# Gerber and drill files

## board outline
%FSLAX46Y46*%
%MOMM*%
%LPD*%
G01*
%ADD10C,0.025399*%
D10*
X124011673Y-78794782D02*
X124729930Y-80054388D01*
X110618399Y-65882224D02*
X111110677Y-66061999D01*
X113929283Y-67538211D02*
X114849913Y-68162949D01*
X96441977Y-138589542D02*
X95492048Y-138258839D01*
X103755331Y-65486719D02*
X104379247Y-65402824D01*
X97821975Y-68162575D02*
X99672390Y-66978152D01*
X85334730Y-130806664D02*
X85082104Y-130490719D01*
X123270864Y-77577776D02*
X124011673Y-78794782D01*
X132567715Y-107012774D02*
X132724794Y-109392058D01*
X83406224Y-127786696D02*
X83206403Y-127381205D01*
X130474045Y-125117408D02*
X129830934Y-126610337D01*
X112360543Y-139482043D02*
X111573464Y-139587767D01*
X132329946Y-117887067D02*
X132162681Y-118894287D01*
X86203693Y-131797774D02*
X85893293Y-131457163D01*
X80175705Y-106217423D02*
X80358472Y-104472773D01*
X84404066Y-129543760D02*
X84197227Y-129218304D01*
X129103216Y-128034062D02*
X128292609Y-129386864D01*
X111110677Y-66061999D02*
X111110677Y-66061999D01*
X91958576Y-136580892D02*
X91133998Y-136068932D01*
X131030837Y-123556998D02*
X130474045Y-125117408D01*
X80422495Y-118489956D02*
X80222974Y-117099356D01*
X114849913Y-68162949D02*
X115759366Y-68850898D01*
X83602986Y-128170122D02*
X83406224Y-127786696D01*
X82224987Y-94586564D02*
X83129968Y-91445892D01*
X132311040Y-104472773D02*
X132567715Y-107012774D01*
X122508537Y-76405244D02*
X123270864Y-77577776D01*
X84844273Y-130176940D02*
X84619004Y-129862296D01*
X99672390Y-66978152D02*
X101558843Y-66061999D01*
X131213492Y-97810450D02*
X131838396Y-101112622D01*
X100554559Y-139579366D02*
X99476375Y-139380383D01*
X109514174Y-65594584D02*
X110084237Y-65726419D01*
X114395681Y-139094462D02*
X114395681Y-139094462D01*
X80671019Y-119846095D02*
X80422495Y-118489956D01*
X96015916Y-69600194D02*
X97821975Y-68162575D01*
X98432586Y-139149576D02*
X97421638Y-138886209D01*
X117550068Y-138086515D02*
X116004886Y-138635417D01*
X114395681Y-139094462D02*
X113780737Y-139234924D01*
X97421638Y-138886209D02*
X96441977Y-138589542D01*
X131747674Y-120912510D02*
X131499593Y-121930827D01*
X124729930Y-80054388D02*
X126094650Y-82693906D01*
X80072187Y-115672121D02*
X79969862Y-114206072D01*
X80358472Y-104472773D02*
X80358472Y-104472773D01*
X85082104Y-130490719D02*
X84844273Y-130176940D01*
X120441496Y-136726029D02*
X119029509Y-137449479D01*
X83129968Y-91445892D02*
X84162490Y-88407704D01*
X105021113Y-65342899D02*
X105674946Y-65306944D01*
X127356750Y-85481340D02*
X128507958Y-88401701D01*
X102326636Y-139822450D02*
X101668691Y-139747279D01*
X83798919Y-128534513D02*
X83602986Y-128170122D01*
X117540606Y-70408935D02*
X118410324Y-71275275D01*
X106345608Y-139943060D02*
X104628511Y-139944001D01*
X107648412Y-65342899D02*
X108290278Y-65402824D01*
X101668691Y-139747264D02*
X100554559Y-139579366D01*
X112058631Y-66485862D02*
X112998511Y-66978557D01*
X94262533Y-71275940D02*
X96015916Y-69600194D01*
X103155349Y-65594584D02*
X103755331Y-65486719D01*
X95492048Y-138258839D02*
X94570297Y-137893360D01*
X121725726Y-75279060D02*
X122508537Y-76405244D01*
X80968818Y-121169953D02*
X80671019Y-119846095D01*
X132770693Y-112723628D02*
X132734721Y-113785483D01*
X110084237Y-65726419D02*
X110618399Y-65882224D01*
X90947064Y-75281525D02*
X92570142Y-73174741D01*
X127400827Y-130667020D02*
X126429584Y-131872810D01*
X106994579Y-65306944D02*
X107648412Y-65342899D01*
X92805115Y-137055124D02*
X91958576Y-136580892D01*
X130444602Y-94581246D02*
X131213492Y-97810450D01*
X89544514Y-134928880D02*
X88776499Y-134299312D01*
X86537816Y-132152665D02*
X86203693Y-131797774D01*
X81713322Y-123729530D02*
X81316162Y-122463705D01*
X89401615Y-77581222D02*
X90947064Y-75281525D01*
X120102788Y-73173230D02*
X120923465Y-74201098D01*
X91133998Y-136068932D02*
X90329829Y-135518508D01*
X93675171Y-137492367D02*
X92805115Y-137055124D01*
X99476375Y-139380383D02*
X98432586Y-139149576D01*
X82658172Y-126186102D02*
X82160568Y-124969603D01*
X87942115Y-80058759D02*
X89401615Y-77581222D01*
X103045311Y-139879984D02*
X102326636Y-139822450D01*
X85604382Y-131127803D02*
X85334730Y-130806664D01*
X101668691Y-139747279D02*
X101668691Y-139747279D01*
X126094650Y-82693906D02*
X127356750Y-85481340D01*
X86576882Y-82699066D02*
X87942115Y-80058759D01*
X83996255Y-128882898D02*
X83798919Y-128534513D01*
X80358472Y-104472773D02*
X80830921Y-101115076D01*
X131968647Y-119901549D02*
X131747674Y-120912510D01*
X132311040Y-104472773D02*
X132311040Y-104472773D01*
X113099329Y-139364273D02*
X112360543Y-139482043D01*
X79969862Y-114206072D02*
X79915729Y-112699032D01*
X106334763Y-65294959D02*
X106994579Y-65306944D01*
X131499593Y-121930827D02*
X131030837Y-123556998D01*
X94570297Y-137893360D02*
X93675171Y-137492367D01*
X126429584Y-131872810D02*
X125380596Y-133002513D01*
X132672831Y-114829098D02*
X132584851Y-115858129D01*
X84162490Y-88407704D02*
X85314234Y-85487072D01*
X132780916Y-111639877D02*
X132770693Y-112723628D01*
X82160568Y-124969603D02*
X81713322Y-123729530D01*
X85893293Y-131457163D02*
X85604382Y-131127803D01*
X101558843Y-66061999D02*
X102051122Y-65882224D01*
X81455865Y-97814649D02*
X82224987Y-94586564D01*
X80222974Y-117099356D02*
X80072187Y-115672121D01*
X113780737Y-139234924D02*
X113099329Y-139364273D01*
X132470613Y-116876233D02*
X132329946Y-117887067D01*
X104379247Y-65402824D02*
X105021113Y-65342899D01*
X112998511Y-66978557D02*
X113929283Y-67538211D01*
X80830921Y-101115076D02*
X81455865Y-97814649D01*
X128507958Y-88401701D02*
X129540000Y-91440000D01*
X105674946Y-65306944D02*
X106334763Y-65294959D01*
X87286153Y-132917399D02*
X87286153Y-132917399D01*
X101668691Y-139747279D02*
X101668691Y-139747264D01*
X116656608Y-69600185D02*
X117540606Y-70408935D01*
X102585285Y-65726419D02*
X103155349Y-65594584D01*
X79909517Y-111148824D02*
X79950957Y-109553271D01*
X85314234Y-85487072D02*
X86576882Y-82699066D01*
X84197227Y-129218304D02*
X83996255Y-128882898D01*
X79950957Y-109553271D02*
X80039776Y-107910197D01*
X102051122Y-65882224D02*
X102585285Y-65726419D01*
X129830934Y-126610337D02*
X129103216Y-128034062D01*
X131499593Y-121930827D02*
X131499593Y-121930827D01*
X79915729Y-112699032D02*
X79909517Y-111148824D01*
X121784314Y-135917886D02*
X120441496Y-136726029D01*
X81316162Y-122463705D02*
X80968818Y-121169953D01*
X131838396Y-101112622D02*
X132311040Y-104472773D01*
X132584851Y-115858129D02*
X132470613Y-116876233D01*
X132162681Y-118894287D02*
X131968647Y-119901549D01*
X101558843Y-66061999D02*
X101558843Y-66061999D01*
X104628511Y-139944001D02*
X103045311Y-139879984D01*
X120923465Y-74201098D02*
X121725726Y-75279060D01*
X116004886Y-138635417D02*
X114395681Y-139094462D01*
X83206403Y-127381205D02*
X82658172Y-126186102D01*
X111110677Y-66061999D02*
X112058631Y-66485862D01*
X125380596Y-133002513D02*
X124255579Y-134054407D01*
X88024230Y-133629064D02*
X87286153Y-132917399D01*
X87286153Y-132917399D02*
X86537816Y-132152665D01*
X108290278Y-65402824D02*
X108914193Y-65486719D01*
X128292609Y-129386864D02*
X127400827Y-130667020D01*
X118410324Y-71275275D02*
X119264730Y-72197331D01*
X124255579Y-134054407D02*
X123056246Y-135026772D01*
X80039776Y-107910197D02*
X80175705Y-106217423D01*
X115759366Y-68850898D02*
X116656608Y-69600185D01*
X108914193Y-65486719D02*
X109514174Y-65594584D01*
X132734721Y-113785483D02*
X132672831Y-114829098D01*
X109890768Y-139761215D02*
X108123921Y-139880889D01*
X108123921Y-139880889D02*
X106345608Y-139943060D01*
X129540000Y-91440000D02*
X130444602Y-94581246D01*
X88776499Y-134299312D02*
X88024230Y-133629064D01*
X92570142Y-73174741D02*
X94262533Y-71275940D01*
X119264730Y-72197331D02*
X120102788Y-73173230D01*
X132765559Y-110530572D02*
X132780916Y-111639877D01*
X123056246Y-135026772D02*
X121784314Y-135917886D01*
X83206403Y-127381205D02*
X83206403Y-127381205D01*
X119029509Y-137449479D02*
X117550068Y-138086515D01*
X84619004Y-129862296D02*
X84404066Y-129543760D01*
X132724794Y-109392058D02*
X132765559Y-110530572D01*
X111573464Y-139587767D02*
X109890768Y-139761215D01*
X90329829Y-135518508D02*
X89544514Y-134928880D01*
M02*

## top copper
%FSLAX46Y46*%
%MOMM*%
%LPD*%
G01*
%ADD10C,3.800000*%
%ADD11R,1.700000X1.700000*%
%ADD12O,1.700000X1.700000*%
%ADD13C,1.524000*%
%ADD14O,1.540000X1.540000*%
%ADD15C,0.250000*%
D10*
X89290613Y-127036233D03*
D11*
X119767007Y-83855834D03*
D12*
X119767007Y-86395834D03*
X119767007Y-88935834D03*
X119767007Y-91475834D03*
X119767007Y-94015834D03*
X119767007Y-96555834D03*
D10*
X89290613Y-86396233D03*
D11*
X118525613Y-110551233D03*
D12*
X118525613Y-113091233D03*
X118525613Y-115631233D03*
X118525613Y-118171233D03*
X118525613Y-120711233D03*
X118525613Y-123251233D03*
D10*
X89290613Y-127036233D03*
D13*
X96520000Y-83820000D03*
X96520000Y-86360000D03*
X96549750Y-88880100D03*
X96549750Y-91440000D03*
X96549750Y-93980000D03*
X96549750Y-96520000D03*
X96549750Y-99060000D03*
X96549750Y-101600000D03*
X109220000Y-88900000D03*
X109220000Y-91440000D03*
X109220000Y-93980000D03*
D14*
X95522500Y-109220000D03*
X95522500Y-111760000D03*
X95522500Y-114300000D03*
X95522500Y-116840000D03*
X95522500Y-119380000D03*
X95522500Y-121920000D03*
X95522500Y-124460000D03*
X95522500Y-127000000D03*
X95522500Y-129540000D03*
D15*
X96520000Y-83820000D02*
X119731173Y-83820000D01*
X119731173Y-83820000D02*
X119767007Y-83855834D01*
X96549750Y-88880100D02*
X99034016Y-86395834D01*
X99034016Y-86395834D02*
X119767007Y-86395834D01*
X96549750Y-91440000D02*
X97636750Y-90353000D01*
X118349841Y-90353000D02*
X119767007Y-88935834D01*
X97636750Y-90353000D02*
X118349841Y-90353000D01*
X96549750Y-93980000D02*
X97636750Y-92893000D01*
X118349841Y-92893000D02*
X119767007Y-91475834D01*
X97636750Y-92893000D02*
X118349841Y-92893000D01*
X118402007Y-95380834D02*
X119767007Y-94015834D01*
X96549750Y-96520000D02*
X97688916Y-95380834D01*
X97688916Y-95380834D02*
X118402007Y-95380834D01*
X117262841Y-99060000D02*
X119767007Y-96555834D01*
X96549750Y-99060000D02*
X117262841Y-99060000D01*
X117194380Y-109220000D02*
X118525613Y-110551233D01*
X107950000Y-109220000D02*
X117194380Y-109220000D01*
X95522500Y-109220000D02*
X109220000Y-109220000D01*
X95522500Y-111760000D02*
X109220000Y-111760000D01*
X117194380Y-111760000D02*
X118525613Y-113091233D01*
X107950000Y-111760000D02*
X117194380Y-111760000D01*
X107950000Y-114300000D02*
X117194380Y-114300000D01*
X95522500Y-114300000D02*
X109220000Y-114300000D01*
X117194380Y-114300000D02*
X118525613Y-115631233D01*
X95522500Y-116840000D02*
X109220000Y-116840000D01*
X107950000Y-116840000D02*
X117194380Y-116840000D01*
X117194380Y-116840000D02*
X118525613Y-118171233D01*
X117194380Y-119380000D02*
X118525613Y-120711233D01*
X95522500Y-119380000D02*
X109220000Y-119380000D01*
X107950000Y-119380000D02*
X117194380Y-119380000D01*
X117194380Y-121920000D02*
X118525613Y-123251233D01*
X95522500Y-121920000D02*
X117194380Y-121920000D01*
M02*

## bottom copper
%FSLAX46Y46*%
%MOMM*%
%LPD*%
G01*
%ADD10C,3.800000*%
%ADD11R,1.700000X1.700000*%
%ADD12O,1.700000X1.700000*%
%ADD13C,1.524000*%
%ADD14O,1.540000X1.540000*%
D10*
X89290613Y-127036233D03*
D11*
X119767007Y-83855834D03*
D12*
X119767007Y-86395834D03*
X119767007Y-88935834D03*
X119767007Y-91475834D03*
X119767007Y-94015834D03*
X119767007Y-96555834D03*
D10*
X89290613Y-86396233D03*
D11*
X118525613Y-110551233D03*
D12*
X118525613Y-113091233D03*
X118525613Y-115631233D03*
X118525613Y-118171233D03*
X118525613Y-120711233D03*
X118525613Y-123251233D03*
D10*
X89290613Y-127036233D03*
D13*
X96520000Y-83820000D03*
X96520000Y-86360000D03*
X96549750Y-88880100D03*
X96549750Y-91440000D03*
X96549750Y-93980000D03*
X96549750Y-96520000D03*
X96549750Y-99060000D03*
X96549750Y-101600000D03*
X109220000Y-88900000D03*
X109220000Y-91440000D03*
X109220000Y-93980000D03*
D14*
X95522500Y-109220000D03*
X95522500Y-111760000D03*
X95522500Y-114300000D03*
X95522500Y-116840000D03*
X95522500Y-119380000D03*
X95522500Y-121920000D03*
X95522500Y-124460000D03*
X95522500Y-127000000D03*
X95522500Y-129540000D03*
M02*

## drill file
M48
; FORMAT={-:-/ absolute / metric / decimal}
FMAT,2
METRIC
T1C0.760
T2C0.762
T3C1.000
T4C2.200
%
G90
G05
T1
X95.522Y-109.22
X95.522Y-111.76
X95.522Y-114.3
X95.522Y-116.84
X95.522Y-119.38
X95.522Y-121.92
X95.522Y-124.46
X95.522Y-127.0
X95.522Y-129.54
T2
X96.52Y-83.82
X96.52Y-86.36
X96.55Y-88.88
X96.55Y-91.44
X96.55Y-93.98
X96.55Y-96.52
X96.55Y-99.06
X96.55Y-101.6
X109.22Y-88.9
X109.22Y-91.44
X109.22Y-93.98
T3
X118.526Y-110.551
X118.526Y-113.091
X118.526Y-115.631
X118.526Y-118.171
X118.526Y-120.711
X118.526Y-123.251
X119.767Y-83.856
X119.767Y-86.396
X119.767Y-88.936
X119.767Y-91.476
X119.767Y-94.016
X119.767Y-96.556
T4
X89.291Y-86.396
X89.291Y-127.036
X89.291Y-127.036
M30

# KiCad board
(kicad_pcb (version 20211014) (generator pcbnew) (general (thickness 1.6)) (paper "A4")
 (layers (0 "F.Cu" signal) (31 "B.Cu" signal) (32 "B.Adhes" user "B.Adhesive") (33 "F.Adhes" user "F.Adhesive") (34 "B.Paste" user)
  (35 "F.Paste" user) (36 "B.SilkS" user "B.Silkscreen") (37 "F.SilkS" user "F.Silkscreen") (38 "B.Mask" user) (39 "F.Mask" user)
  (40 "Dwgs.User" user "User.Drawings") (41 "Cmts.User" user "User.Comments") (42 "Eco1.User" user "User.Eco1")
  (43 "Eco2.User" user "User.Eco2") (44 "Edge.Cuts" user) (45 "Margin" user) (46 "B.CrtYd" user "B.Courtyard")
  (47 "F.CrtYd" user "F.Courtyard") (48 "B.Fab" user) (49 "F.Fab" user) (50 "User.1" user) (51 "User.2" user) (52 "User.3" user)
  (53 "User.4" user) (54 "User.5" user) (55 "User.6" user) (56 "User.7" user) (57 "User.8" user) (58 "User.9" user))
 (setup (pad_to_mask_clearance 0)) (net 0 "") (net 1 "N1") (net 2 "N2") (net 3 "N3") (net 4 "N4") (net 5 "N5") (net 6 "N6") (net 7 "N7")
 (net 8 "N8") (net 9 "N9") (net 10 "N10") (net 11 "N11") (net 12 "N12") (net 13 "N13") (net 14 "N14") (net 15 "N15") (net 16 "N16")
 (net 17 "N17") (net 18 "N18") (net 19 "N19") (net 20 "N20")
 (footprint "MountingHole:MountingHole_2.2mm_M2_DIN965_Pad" (layer "F.Cu") (at 89.290613 127.036233)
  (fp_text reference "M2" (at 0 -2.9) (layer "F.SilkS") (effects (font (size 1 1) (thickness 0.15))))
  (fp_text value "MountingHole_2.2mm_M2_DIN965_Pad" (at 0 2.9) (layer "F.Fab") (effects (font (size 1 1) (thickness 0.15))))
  (pad "1" thru_hole circle (at 0 0) (size 3.8 3.8) (drill 2.2) (layers *.Cu *.Mask)))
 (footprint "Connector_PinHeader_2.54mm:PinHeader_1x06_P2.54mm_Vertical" (layer "F.Cu") (at 119.767007 83.855834)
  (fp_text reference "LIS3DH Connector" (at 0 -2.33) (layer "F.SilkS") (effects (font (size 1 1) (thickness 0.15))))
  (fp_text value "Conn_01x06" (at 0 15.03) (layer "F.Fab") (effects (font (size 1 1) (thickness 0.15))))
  (pad "1" thru_hole rect (at 0 0) (size 1.7 1.7) (drill 1) (layers *.Cu *.Mask) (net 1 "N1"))
  (pad "2" thru_hole oval (at 0 2.54) (size 1.7 1.7) (drill 1) (layers *.Cu *.Mask) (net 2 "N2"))
  (pad "3" thru_hole oval (at 0 5.08) (size 1.7 1.7) (drill 1) (layers *.Cu *.Mask) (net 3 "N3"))
  (pad "4" thru_hole oval (at 0 7.62) (size 1.7 1.7) (drill 1) (layers *.Cu *.Mask) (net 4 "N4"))
  (pad "5" thru_hole oval (at 0 10.16) (size 1.7 1.7) (drill 1) (layers *.Cu *.Mask) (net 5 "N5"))
  (pad "6" thru_hole oval (at 0 12.7) (size 1.7 1.7) (drill 1) (layers *.Cu *.Mask) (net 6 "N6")))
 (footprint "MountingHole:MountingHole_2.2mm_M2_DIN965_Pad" (layer "F.Cu") (at 89.290613 86.396233)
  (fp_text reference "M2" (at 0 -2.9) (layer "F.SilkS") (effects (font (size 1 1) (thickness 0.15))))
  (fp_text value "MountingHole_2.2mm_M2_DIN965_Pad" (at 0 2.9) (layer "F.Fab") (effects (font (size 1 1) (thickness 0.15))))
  (pad "1" thru_hole circle (at 0 0) (size 3.8 3.8) (drill 2.2) (layers *.Cu *.Mask)))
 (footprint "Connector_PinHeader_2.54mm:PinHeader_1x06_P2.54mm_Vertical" (layer "F.Cu") (at 118.525613 110.551233)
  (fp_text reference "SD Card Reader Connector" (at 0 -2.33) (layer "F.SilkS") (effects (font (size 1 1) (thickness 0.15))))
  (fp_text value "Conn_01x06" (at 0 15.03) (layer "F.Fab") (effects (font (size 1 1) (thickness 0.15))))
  (pad "1" thru_hole rect (at 0 0) (size 1.7 1.7) (drill 1) (layers *.Cu *.Mask) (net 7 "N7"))
  (pad "2" thru_hole oval (at 0 2.54) (size 1.7 1.7) (drill 1) (layers *.Cu *.Mask) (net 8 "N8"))
  (pad "3" thru_hole oval (at 0 5.08) (size 1.7 1.7) (drill 1) (layers *.Cu *.Mask) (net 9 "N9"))
  (pad "4" thru_hole oval (at 0 7.62) (size 1.7 1.7) (drill 1) (layers *.Cu *.Mask) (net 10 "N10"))
  (pad "5" thru_hole oval (at 0 10.16) (size 1.7 1.7) (drill 1) (layers *.Cu *.Mask) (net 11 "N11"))
  (pad "6" thru_hole oval (at 0 12.7) (size 1.7 1.7) (drill 1) (layers *.Cu *.Mask) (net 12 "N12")))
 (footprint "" (layer "F.Cu") (at 89.290613 127.036233)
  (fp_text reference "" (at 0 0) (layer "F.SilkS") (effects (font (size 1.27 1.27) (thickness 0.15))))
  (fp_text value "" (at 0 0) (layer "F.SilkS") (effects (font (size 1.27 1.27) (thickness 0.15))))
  (pad "1" thru_hole circle (at 0 0) (size 3.8 3.8) (drill 2.2) (layers *.Cu *.Mask)))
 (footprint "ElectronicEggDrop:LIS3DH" (layer "B.Cu") (at 104.14 78.74 180)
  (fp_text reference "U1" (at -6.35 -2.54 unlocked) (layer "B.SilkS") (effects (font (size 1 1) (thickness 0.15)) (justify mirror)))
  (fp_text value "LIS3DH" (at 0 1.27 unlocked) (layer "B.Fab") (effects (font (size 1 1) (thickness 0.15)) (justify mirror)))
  (pad "1" thru_hole circle (at 7.62 -5.08 180) (size 1.524 1.524) (drill 0.762) (layers *.Cu *.Mask) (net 1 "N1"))
  (pad "2" thru_hole circle (at 7.62 -7.62 180) (size 1.524 1.524) (drill 0.762) (layers *.Cu *.Mask) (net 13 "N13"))
  (pad "3" thru_hole circle (at 7.59025 -10.1401 180) (size 1.524 1.524) (drill 0.762) (layers *.Cu *.Mask) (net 2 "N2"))
  (pad "4" thru_hole circle (at 7.59025 -12.7 180) (size 1.524 1.524) (drill 0.762) (layers *.Cu *.Mask) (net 3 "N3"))
  (pad "5" thru_hole circle (at 7.59025 -15.24 180) (size 1.524 1.524) (drill 0.762) (layers *.Cu *.Mask) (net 4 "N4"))
  (pad "6" thru_hole circle (at 7.59025 -17.78 180) (size 1.524 1.524) (drill 0.762) (layers *.Cu *.Mask) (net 5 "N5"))
  (pad "7" thru_hole circle (at 7.59025 -20.32 180) (size 1.524 1.524) (drill 0.762) (layers *.Cu *.Mask) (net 6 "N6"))
  (pad "8" thru_hole circle (at 7.59025 -22.86 180) (size 1.524 1.524) (drill 0.762) (layers *.Cu *.Mask) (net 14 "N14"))
  (pad "9" thru_hole circle (at -5.08 -10.16 180) (size 1.524 1.524) (drill 0.762) (layers *.Cu *.Mask) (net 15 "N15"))
  (pad "10" thru_hole circle (at -5.08 -12.7 180) (size 1.524 1.524) (drill 0.762) (layers *.Cu *.Mask) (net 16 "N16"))
  (pad "11" thru_hole circle (at -5.08 -15.24 180) (size 1.524 1.524) (drill 0.762) (layers *.Cu *.Mask) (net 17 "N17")))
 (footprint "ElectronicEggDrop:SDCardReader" (layer "B.Cu") (at 94.2525 119.38 -90)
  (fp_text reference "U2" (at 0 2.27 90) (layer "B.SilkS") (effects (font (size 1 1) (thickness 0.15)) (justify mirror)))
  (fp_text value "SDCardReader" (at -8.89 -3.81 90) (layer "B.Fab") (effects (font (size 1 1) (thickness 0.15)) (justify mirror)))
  (pad "1" thru_hole oval (at -10.16 -1.27 270) (size 1.54 1.54) (drill 0.76) (layers *.Cu *.Mask) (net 7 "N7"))
  (pad "2" thru_hole oval (at -7.62 -1.27 270) (size 1.54 1.54) (drill 0.76) (layers *.Cu *.Mask) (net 8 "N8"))
  (pad "3" thru_hole oval (at -5.08 -1.27 270) (size 1.54 1.54) (drill 0.76) (layers *.Cu *.Mask) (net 9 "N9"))
  (pad "4" thru_hole oval (at -2.54 -1.27 270) (size 1.54 1.54) (drill 0.76) (layers *.Cu *.Mask) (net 10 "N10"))
  (pad "5" thru_hole oval (at 0 -1.27 270) (size 1.54 1.54) (drill 0.76) (layers *.Cu *.Mask) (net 11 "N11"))
  (pad "6" thru_hole oval (at 2.54 -1.27 270) (size 1.54 1.54) (drill 0.76) (layers *.Cu *.Mask) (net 12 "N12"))
  (pad "7" thru_hole oval (at 5.08 -1.27 270) (size 1.54 1.54) (drill 0.76) (layers *.Cu *.Mask) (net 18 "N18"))
  (pad "8" thru_hole oval (at 7.62 -1.27 270) (size 1.54 1.54) (drill 0.76) (layers *.Cu *.Mask) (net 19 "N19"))
  (pad "9" thru_hole oval (at 10.16 -1.27 270) (size 1.54 1.54) (drill 0.76) (layers *.Cu *.Mask) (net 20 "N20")))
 (gr_line (start 124.011673 78.794782) (end 124.72993 80.054388) (layer "Edge.Cuts") (width 0.025399))
 (gr_line (start 110.618399 65.882224) (end 111.110677 66.061999) (layer "Edge.Cuts") (width 0.025399))
 (gr_line (start 113.929283 67.538211) (end 114.849913 68.162949) (layer "Edge.Cuts") (width 0.025399))
 (gr_line (start 96.441977 138.589542) (end 95.492048 138.258839) (layer "Edge.Cuts") (width 0.025399))
 (gr_line (start 103.755331 65.486719) (end 104.379247 65.402824) (layer "Edge.Cuts") (width 0.025399))
 (gr_line (start 97.821975 68.162575) (end 99.67239 66.978152) (layer "Edge.Cuts") (width 0.025399))
 (gr_line (start 85.33473 130.806664) (end 85.082104 130.490719) (layer "Edge.Cuts") (width 0.025399))
 (gr_line (start 123.270864 77.577776) (end 124.011673 78.794782) (layer "Edge.Cuts") (width 0.025399))
 (gr_line (start 132.567715 107.012774) (end 132.724794 109.392058) (layer "Edge.Cuts") (width 0.025399))
 (gr_line (start 83.406224 127.786696) (end 83.206403 127.381205) (layer "Edge.Cuts") (width 0.025399))
 (gr_line (start 130.474045 125.117408) (end 129.830934 126.610337) (layer "Edge.Cuts") (width 0.025399))
 (gr_line (start 112.360543 139.482043) (end 111.573464 139.587767) (layer "Edge.Cuts") (width 0.025399))
 (gr_line (start 132.329946 117.887067) (end 132.162681 118.894287) (layer "Edge.Cuts") (width 0.025399))
 (gr_line (start 86.203693 131.797774) (end 85.893293 131.457163) (layer "Edge.Cuts") (width 0.025399))
 (gr_line (start 80.175705 106.217423) (end 80.358472 104.472773) (layer "Edge.Cuts") (width 0.025399))
 (gr_line (start 84.404066 129.54376) (end 84.197227 129.218304) (layer "Edge.Cuts") (width 0.025399))
 (gr_line (start 129.103216 128.034062) (end 128.292609 129.386864) (layer "Edge.Cuts") (width 0.025399))
 (gr_line (start 111.110677 66.061999) (end 111.110677 66.061999) (layer "Edge.Cuts") (width 0.025399))
 (gr_line (start 91.958576 136.580892) (end 91.133998 136.068932) (layer "Edge.Cuts") (width 0.025399))
 (gr_line (start 131.030837 123.556998) (end 130.474045 125.117408) (layer "Edge.Cuts") (width 0.025399))
 (gr_line (start 80.422495 118.489956) (end 80.222974 117.099356) (layer "Edge.Cuts") (width 0.025399))
 (gr_line (start 114.849913 68.162949) (end 115.759366 68.850898) (layer "Edge.Cuts") (width 0.025399))
 (gr_line (start 83.602986 128.170122) (end 83.406224 127.786696) (layer "Edge.Cuts") (width 0.025399))
 (gr_line (start 82.224987 94.586564) (end 83.129968 91.445892) (layer "Edge.Cuts") (width 0.025399))
 (gr_line (start 132.31104 104.472773) (end 132.567715 107.012774) (layer "Edge.Cuts") (width 0.025399))
 (gr_line (start 122.508537 76.405244) (end 123.270864 77.577776) (layer "Edge.Cuts") (width 0.025399))
 (gr_line (start 84.844273 130.17694) (end 84.619004 129.862296) (layer "Edge.Cuts") (width 0.025399))
 (gr_line (start 99.67239 66.978152) (end 101.558843 66.061999) (layer "Edge.Cuts") (width 0.025399))
 (gr_line (start 131.213492 97.81045) (end 131.838396 101.112622) (layer "Edge.Cuts") (width 0.025399))
 (gr_line (start 100.554559 139.579366) (end 99.476375 139.380383) (layer "Edge.Cuts") (width 0.025399))
 (gr_line (start 109.514174 65.594584) (end 110.084237 65.726419) (layer "Edge.Cuts") (width 0.025399))
 (gr_line (start 114.395681 139.094462) (end 114.395681 139.094462) (layer "Edge.Cuts") (width 0.025399))
 (gr_line (start 80.671019 119.846095) (end 80.422495 118.489956) (layer "Edge.Cuts") (width 0.025399))
 (gr_line (start 96.015916 69.600194) (end 97.821975 68.162575) (layer "Edge.Cuts") (width 0.025399))
 (gr_line (start 98.432586 139.149576) (end 97.421638 138.886209) (layer "Edge.Cuts") (width 0.025399))
 (gr_line (start 117.550068 138.086515) (end 116.004886 138.635417) (layer "Edge.Cuts") (width 0.025399))
 (gr_line (start 114.395681 139.094462) (end 113.780737 139.234924) (layer "Edge.Cuts") (width 0.025399))
 (gr_line (start 97.421638 138.886209) (end 96.441977 138.589542) (layer "Edge.Cuts") (width 0.025399))
 (gr_line (start 131.747674 120.91251) (end 131.499593 121.930827) (layer "Edge.Cuts") (width 0.025399))
 (gr_line (start 124.72993 80.054388) (end 126.09465 82.693906) (layer "Edge.Cuts") (width 0.025399))
 (gr_line (start 80.072187 115.672121) (end 79.969862 114.206072) (layer "Edge.Cuts") (width 0.025399))
 (gr_line (start 80.358472 104.472773) (end 80.358472 104.472773) (layer "Edge.Cuts") (width 0.025399))
 (gr_line (start 85.082104 130.490719) (end 84.844273 130.17694) (layer "Edge.Cuts") (width 0.025399))
 (gr_line (start 120.441496 136.726029) (end 119.029509 137.449479) (layer "Edge.Cuts") (width 0.025399))
 (gr_line (start 83.129968 91.445892) (end 84.16249 88.407704) (layer "Edge.Cuts") (width 0.025399))
 (gr_line (start 105.021113 65.342899) (end 105.674946 65.306944) (layer "Edge.Cuts") (width 0.025399))
 (gr_line (start 127.35675 85.48134) (end 128.507958 88.401701) (layer "Edge.Cuts") (width 0.025399))
 (gr_line (start 102.326636 139.82245) (end 101.668691 139.747279) (layer "Edge.Cuts") (width 0.025399))
 (gr_line (start 83.798919 128.534513) (end 83.602986 128.170122) (layer "Edge.Cuts") (width 0.025399))
 (gr_line (start 117.540606 70.408935) (end 118.410324 71.275275) (layer "Edge.Cuts") (width 0.025399))
 (gr_line (start 106.345608 139.94306) (end 104.628511 139.944001) (layer "Edge.Cuts") (width 0.025399))
 (gr_line (start 107.648412 65.342899) (end 108.290278 65.402824) (layer "Edge.Cuts") (width 0.025399))
 (gr_line (start 101.668691 139.747264) (end 100.554559 139.579366) (layer "Edge.Cuts") (width 0.025399))
 (gr_line (start 112.058631 66.485862) (end 112.998511 66.978557) (layer "Edge.Cuts") (width 0.025399))
 (gr_line (start 94.262533 71.27594) (end 96.015916 69.600194) (layer "Edge.Cuts") (width 0.025399))
 (gr_line (start 103.155349 65.594584) (end 103.755331 65.486719) (layer "Edge.Cuts") (width 0.025399))
 (gr_line (start 95.492048 138.258839) (end 94.570297 137.89336) (layer "Edge.Cuts") (width 0.025399))
 (gr_line (start 121.725726 75.27906) (end 122.508537 76.405244) (layer "Edge.Cuts") (width 0.025399))
 (gr_line (start 80.968818 121.169953) (end 80.671019 119.846095) (layer "Edge.Cuts") (width 0.025399))
 (gr_line (start 132.770693 112.723628) (end 132.734721 113.785483) (layer "Edge.Cuts") (width 0.025399))
 (gr_line (start 110.084237 65.726419) (end 110.618399 65.882224) (layer "Edge.Cuts") (width 0.025399))
 (gr_line (start 90.947064 75.281525) (end 92.570142 73.174741) (layer "Edge.Cuts") (width 0.025399))
 (gr_line (start 127.400827 130.66702) (end 126.429584 131.87281) (layer "Edge.Cuts") (width 0.025399))
 (gr_line (start 106.994579 65.306944) (end 107.648412 65.342899) (layer "Edge.Cuts") (width 0.025399))
 (gr_line (start 92.805115 137.055124) (end 91.958576 136.580892) (layer "Edge.Cuts") (width 0.025399))
 (gr_line (start 130.444602 94.581246) (end 131.213492 97.81045) (layer "Edge.Cuts") (width 0.025399))
 (gr_line (start 89.544514 134.92888) (end 88.776499 134.299312) (layer "Edge.Cuts") (width 0.025399))
 (gr_line (start 86.537816 132.152665) (end 86.203693 131.797774) (layer "Edge.Cuts") (width 0.025399))
 (gr_line (start 81.713322 123.72953) (end 81.316162 122.463705) (layer "Edge.Cuts") (width 0.025399))
 (gr_line (start 89.401615 77.581222) (end 90.947064 75.281525) (layer "Edge.Cuts") (width 0.025399))
 (gr_line (start 120.102788 73.17323) (end 120.923465 74.201098) (layer "Edge.Cuts") (width 0.025399))
 (gr_line (start 91.133998 136.068932) (end 90.329829 135.518508) (layer "Edge.Cuts") (width 0.025399))
 (gr_line (start 93.675171 137.492367) (end 92.805115 137.055124) (layer "Edge.Cuts") (width 0.025399))
 (gr_line (start 99.476375 139.380383) (end 98.432586 139.149576) (layer "Edge.Cuts") (width 0.025399))
 (gr_line (start 82.658172 126.186102) (end 82.160568 124.969603) (layer "Edge.Cuts") (width 0.025399))
 (gr_line (start 87.942115 80.058759) (end 89.401615 77.581222) (layer "Edge.Cuts") (width 0.025399))
 (gr_line (start 103.045311 139.879984) (end 102.326636 139.82245) (layer "Edge.Cuts") (width 0.025399))
 (gr_line (start 85.604382 131.127803) (end 85.33473 130.806664) (layer "Edge.Cuts") (width 0.025399))
 (gr_line (start 101.668691 139.747279) (end 101.668691 139.747279) (layer "Edge.Cuts") (width 0.025399))
 (gr_line (start 126.09465 82.693906) (end 127.35675 85.48134) (layer "Edge.Cuts") (width 0.025399))
 (gr_line (start 86.576882 82.699066) (end 87.942115 80.058759) (layer "Edge.Cuts") (width 0.025399))
 (gr_line (start 83.996255 128.882898) (end 83.798919 128.534513) (layer "Edge.Cuts") (width 0.025399))
 (gr_line (start 80.358472 104.472773) (end 80.830921 101.115076) (layer "Edge.Cuts") (width 0.025399))
 (gr_line (start 131.968647 119.901549) (end 131.747674 120.91251) (layer "Edge.Cuts") (width 0.025399))
 (gr_line (start 132.31104 104.472773) (end 132.31104 104.472773) (layer "Edge.Cuts") (width 0.025399))
 (gr_line (start 113.099329 139.364273) (end 112.360543 139.482043) (layer "Edge.Cuts") (width 0.025399))
 (gr_line (start 79.969862 114.206072) (end 79.915729 112.699032) (layer "Edge.Cuts") (width 0.025399))
 (gr_line (start 106.334763 65.294959) (end 106.994579 65.306944) (layer "Edge.Cuts") (width 0.025399))
 (gr_line (start 131.499593 121.930827) (end 131.030837 123.556998) (layer "Edge.Cuts") (width 0.025399))
 (gr_line (start 94.570297 137.89336) (end 93.675171 137.492367) (layer "Edge.Cuts") (width 0.025399))
 (gr_line (start 126.429584 131.87281) (end 125.380596 133.002513) (layer "Edge.Cuts") (width 0.025399))
 (gr_line (start 132.672831 114.829098) (end 132.584851 115.858129) (layer "Edge.Cuts") (width 0.025399))
 (gr_line (start 84.16249 88.407704) (end 85.314234 85.487072) (layer "Edge.Cuts") (width 0.025399))
 (gr_line (start 132.780916 111.639877) (end 132.770693 112.723628) (layer "Edge.Cuts") (width 0.025399))
 (gr_line (start 82.160568 124.969603) (end 81.713322 123.72953) (layer "Edge.Cuts") (width 0.025399))
 (gr_line (start 85.893293 131.457163) (end 85.604382 131.127803) (layer "Edge.Cuts") (width 0.025399))
 (gr_line (start 101.558843 66.061999) (end 102.051122 65.882224) (layer "Edge.Cuts") (width 0.025399))
 (gr_line (start 81.455865 97.814649) (end 82.224987 94.586564) (layer "Edge.Cuts") (width 0.025399))
 (gr_line (start 80.222974 117.099356) (end 80.072187 115.672121) (layer "Edge.Cuts") (width 0.025399))
 (gr_line (start 113.780737 139.234924) (end 113.099329 139.364273) (layer "Edge.Cuts") (width 0.025399))
 (gr_line (start 132.470613 116.876233) (end 132.329946 117.887067) (layer "Edge.Cuts") (width 0.025399))
 (gr_line (start 104.379247 65.402824) (end 105.021113 65.342899) (layer "Edge.Cuts") (width 0.025399))
 (gr_line (start 112.998511 66.978557) (end 113.929283 67.538211) (layer "Edge.Cuts") (width 0.025399))
 (gr_line (start 80.830921 101.115076) (end 81.455865 97.814649) (layer "Edge.Cuts") (width 0.025399))
 (gr_line (start 128.507958 88.401701) (end 129.54 91.44) (layer "Edge.Cuts") (width 0.025399))
 (gr_line (start 105.674946 65.306944) (end 106.334763 65.294959) (layer "Edge.Cuts") (width 0.025399))
 (gr_line (start 87.286153 132.917399) (end 87.286153 132.917399) (layer "Edge.Cuts") (width 0.025399))
 (gr_line (start 101.668691 139.747279) (end 101.668691 139.747264) (layer "Edge.Cuts") (width 0.025399))
 (gr_line (start 116.656608 69.600185) (end 117.540606 70.408935) (layer "Edge.Cuts") (width 0.025399))
 (gr_line (start 102.585285 65.726419) (end 103.155349 65.594584) (layer "Edge.Cuts") (width 0.025399))
 (gr_line (start 79.909517 111.148824) (end 79.950957 109.553271) (layer "Edge.Cuts") (width 0.025399))
 (gr_line (start 85.314234 85.487072) (end 86.576882 82.699066) (layer "Edge.Cuts") (width 0.025399))
 (gr_line (start 84.197227 129.218304) (end 83.996255 128.882898) (layer "Edge.Cuts") (width 0.025399))
 (gr_line (start 79.950957 109.553271) (end 80.039776 107.910197) (layer "Edge.Cuts") (width 0.025399))
 (gr_line (start 102.051122 65.882224) (end 102.585285 65.726419) (layer "Edge.Cuts") (width 0.025399))
 (gr_line (start 129.830934 126.610337) (end 129.103216 128.034062) (layer "Edge.Cuts") (width 0.025399))
 (gr_line (start 131.499593 121.930827) (end 131.499593 121.930827) (layer "Edge.Cuts") (width 0.025399))
 (gr_line (start 79.915729 112.699032) (end 79.909517 111.148824) (layer "Edge.Cuts") (width 0.025399))
 (gr_line (start 121.784314 135.917886) (end 120.441496 136.726029) (layer "Edge.Cuts") (width 0.025399))
 (gr_line (start 81.316162 122.463705) (end 80.968818 121.169953) (layer "Edge.Cuts") (width 0.025399))
 (gr_line (start 131.838396 101.112622) (end 132.31104 104.472773) (layer "Edge.Cuts") (width 0.025399))
 (gr_line (start 132.584851 115.858129) (end 132.470613 116.876233) (layer "Edge.Cuts") (width 0.025399))
 (gr_line (start 132.162681 118.894287) (end 131.968647 119.901549) (layer "Edge.Cuts") (width 0.025399))
 (gr_line (start 101.558843 66.061999) (end 101.558843 66.061999) (layer "Edge.Cuts") (width 0.025399))
 (gr_line (start 104.628511 139.944001) (end 103.045311 139.879984) (layer "Edge.Cuts") (width 0.025399))
 (gr_line (start 120.923465 74.201098) (end 121.725726 75.27906) (layer "Edge.Cuts") (width 0.025399))
 (gr_line (start 116.004886 138.635417) (end 114.395681 139.094462) (layer "Edge.Cuts") (width 0.025399))
 (gr_line (start 83.206403 127.381205) (end 82.658172 126.186102) (layer "Edge.Cuts") (width 0.025399))
 (gr_line (start 111.110677 66.061999) (end 112.058631 66.485862) (layer "Edge.Cuts") (width 0.025399))
 (gr_line (start 125.380596 133.002513) (end 124.255579 134.054407) (layer "Edge.Cuts") (width 0.025399))
 (gr_line (start 88.02423 133.629064) (end 87.286153 132.917399) (layer "Edge.Cuts") (width 0.025399))
 (gr_line (start 87.286153 132.917399) (end 86.537816 132.152665) (layer "Edge.Cuts") (width 0.025399))
 (gr_line (start 108.290278 65.402824) (end 108.914193 65.486719) (layer "Edge.Cuts") (width 0.025399))
 (gr_line (start 128.292609 129.386864) (end 127.400827 130.66702) (layer "Edge.Cuts") (width 0.025399))
 (gr_line (start 118.410324 71.275275) (end 119.26473 72.197331) (layer "Edge.Cuts") (width 0.025399))
 (gr_line (start 124.255579 134.054407) (end 123.056246 135.026772) (layer "Edge.Cuts") (width 0.025399))
 (gr_line (start 80.039776 107.910197) (end 80.175705 106.217423) (layer "Edge.Cuts") (width 0.025399))
 (gr_line (start 115.759366 68.850898) (end 116.656608 69.600185) (layer "Edge.Cuts") (width 0.025399))
 (gr_line (start 108.914193 65.486719) (end 109.514174 65.594584) (layer "Edge.Cuts") (width 0.025399))
 (gr_line (start 132.734721 113.785483) (end 132.672831 114.829098) (layer "Edge.Cuts") (width 0.025399))
 (gr_line (start 109.890768 139.761215) (end 108.123921 139.880889) (layer "Edge.Cuts") (width 0.025399))
 (gr_line (start 108.123921 139.880889) (end 106.345608 139.94306) (layer "Edge.Cuts") (width 0.025399))
 (gr_line (start 129.54 91.44) (end 130.444602 94.581246) (layer "Edge.Cuts") (width 0.025399))
 (gr_line (start 88.776499 134.299312) (end 88.02423 133.629064) (layer "Edge.Cuts") (width 0.025399))
 (gr_line (start 92.570142 73.174741) (end 94.262533 71.27594) (layer "Edge.Cuts") (width 0.025399))
 (gr_line (start 119.26473 72.197331) (end 120.102788 73.17323) (layer "Edge.Cuts") (width 0.025399))
 (gr_line (start 132.765559 110.530572) (end 132.780916 111.639877) (layer "Edge.Cuts") (width 0.025399))
 (gr_line (start 123.056246 135.026772) (end 121.784314 135.917886) (layer "Edge.Cuts") (width 0.025399))
 (gr_line (start 83.206403 127.381205) (end 83.206403 127.381205) (layer "Edge.Cuts") (width 0.025399))
 (gr_line (start 119.029509 137.449479) (end 117.550068 138.086515) (layer "Edge.Cuts") (width 0.025399))
 (gr_line (start 84.619004 129.862296) (end 84.404066 129.54376) (layer "Edge.Cuts") (width 0.025399))
 (gr_line (start 132.724794 109.392058) (end 132.765559 110.530572) (layer "Edge.Cuts") (width 0.025399))
 (gr_line (start 111.573464 139.587767) (end 109.890768 139.761215) (layer "Edge.Cuts") (width 0.025399))
 (gr_line (start 90.329829 135.518508) (end 89.544514 134.92888) (layer "Edge.Cuts") (width 0.025399))
 (segment (start 96.52 83.82) (end 119.731173 83.82) (width 0.25) (layer "F.Cu") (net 1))
 (segment (start 119.731173 83.82) (end 119.767007 83.855834) (width 0.25) (layer "F.Cu") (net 1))
 (segment (start 96.54975 88.8801) (end 99.034016 86.395834) (width 0.25) (layer "F.Cu") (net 2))
 (segment (start 99.034016 86.395834) (end 119.767007 86.395834) (width 0.25) (layer "F.Cu") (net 2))
 (segment (start 96.54975 91.44) (end 97.63675 90.353) (width 0.25) (layer "F.Cu") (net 3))
 (segment (start 118.349841 90.353) (end 119.767007 88.935834) (width 0.25) (layer "F.Cu") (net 3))
 (segment (start 97.63675 90.353) (end 118.349841 90.353) (width 0.25) (layer "F.Cu") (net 3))
 (segment (start 96.54975 93.98) (end 97.63675 92.893) (width 0.25) (layer "F.Cu") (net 4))
 (segment (start 118.349841 92.893) (end 119.767007 91.475834) (width 0.25) (layer "F.Cu") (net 4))
 (segment (start 97.63675 92.893) (end 118.349841 92.893) (width 0.25) (layer "F.Cu") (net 4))
 (segment (start 118.402007 95.380834) (end 119.767007 94.015834) (width 0.25) (layer "F.Cu") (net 5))
 (segment (start 96.54975 96.52) (end 97.688916 95.380834) (width 0.25) (layer "F.Cu") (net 5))
 (segment (start 97.688916 95.380834) (end 118.402007 95.380834) (width 0.25) (layer "F.Cu") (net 5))
 (segment (start 117.262841 99.06) (end 119.767007 96.555834) (width 0.25) (layer "F.Cu") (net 6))
 (segment (start 96.54975 99.06) (end 117.262841 99.06) (width 0.25) (layer "F.Cu") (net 6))
 (segment (start 117.19438 109.22) (end 118.525613 110.551233) (width 0.25) (layer "F.Cu") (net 7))
 (segment (start 107.95 109.22) (end 117.19438 109.22) (width 0.25) (layer "F.Cu") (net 7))
 (segment (start 95.5225 109.22) (end 109.22 109.22) (width 0.25) (layer "F.Cu") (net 7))
 (segment (start 95.5225 111.76) (end 109.22 111.76) (width 0.25) (layer "F.Cu") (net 8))
 (segment (start 117.19438 111.76) (end 118.525613 113.091233) (width 0.25) (layer "F.Cu") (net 8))
 (segment (start 107.95 111.76) (end 117.19438 111.76) (width 0.25) (layer "F.Cu") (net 8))
 (segment (start 107.95 114.3) (end 117.19438 114.3) (width 0.25) (layer "F.Cu") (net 9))
 (segment (start 95.5225 114.3) (end 109.22 114.3) (width 0.25) (layer "F.Cu") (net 9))
 (segment (start 117.19438 114.3) (end 118.525613 115.631233) (width 0.25) (layer "F.Cu") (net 9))
 (segment (start 95.5225 116.84) (end 109.22 116.84) (width 0.25) (layer "F.Cu") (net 10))
 (segment (start 107.95 116.84) (end 117.19438 116.84) (width 0.25) (layer "F.Cu") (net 10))
 (segment (start 117.19438 116.84) (end 118.525613 118.171233) (width 0.25) (layer "F.Cu") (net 10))
 (segment (start 117.19438 119.38) (end 118.525613 120.711233) (width 0.25) (layer "F.Cu") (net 11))
 (segment (start 95.5225 119.38) (end 109.22 119.38) (width 0.25) (layer "F.Cu") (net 11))
 (segment (start 107.95 119.38) (end 117.19438 119.38) (width 0.25) (layer "F.Cu") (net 11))
 (segment (start 117.19438 121.92) (end 118.525613 123.251233) (width 0.25) (layer "F.Cu") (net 12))
 (segment (start 95.5225 121.92) (end 117.19438 121.92) (width 0.25) (layer "F.Cu") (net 12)))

